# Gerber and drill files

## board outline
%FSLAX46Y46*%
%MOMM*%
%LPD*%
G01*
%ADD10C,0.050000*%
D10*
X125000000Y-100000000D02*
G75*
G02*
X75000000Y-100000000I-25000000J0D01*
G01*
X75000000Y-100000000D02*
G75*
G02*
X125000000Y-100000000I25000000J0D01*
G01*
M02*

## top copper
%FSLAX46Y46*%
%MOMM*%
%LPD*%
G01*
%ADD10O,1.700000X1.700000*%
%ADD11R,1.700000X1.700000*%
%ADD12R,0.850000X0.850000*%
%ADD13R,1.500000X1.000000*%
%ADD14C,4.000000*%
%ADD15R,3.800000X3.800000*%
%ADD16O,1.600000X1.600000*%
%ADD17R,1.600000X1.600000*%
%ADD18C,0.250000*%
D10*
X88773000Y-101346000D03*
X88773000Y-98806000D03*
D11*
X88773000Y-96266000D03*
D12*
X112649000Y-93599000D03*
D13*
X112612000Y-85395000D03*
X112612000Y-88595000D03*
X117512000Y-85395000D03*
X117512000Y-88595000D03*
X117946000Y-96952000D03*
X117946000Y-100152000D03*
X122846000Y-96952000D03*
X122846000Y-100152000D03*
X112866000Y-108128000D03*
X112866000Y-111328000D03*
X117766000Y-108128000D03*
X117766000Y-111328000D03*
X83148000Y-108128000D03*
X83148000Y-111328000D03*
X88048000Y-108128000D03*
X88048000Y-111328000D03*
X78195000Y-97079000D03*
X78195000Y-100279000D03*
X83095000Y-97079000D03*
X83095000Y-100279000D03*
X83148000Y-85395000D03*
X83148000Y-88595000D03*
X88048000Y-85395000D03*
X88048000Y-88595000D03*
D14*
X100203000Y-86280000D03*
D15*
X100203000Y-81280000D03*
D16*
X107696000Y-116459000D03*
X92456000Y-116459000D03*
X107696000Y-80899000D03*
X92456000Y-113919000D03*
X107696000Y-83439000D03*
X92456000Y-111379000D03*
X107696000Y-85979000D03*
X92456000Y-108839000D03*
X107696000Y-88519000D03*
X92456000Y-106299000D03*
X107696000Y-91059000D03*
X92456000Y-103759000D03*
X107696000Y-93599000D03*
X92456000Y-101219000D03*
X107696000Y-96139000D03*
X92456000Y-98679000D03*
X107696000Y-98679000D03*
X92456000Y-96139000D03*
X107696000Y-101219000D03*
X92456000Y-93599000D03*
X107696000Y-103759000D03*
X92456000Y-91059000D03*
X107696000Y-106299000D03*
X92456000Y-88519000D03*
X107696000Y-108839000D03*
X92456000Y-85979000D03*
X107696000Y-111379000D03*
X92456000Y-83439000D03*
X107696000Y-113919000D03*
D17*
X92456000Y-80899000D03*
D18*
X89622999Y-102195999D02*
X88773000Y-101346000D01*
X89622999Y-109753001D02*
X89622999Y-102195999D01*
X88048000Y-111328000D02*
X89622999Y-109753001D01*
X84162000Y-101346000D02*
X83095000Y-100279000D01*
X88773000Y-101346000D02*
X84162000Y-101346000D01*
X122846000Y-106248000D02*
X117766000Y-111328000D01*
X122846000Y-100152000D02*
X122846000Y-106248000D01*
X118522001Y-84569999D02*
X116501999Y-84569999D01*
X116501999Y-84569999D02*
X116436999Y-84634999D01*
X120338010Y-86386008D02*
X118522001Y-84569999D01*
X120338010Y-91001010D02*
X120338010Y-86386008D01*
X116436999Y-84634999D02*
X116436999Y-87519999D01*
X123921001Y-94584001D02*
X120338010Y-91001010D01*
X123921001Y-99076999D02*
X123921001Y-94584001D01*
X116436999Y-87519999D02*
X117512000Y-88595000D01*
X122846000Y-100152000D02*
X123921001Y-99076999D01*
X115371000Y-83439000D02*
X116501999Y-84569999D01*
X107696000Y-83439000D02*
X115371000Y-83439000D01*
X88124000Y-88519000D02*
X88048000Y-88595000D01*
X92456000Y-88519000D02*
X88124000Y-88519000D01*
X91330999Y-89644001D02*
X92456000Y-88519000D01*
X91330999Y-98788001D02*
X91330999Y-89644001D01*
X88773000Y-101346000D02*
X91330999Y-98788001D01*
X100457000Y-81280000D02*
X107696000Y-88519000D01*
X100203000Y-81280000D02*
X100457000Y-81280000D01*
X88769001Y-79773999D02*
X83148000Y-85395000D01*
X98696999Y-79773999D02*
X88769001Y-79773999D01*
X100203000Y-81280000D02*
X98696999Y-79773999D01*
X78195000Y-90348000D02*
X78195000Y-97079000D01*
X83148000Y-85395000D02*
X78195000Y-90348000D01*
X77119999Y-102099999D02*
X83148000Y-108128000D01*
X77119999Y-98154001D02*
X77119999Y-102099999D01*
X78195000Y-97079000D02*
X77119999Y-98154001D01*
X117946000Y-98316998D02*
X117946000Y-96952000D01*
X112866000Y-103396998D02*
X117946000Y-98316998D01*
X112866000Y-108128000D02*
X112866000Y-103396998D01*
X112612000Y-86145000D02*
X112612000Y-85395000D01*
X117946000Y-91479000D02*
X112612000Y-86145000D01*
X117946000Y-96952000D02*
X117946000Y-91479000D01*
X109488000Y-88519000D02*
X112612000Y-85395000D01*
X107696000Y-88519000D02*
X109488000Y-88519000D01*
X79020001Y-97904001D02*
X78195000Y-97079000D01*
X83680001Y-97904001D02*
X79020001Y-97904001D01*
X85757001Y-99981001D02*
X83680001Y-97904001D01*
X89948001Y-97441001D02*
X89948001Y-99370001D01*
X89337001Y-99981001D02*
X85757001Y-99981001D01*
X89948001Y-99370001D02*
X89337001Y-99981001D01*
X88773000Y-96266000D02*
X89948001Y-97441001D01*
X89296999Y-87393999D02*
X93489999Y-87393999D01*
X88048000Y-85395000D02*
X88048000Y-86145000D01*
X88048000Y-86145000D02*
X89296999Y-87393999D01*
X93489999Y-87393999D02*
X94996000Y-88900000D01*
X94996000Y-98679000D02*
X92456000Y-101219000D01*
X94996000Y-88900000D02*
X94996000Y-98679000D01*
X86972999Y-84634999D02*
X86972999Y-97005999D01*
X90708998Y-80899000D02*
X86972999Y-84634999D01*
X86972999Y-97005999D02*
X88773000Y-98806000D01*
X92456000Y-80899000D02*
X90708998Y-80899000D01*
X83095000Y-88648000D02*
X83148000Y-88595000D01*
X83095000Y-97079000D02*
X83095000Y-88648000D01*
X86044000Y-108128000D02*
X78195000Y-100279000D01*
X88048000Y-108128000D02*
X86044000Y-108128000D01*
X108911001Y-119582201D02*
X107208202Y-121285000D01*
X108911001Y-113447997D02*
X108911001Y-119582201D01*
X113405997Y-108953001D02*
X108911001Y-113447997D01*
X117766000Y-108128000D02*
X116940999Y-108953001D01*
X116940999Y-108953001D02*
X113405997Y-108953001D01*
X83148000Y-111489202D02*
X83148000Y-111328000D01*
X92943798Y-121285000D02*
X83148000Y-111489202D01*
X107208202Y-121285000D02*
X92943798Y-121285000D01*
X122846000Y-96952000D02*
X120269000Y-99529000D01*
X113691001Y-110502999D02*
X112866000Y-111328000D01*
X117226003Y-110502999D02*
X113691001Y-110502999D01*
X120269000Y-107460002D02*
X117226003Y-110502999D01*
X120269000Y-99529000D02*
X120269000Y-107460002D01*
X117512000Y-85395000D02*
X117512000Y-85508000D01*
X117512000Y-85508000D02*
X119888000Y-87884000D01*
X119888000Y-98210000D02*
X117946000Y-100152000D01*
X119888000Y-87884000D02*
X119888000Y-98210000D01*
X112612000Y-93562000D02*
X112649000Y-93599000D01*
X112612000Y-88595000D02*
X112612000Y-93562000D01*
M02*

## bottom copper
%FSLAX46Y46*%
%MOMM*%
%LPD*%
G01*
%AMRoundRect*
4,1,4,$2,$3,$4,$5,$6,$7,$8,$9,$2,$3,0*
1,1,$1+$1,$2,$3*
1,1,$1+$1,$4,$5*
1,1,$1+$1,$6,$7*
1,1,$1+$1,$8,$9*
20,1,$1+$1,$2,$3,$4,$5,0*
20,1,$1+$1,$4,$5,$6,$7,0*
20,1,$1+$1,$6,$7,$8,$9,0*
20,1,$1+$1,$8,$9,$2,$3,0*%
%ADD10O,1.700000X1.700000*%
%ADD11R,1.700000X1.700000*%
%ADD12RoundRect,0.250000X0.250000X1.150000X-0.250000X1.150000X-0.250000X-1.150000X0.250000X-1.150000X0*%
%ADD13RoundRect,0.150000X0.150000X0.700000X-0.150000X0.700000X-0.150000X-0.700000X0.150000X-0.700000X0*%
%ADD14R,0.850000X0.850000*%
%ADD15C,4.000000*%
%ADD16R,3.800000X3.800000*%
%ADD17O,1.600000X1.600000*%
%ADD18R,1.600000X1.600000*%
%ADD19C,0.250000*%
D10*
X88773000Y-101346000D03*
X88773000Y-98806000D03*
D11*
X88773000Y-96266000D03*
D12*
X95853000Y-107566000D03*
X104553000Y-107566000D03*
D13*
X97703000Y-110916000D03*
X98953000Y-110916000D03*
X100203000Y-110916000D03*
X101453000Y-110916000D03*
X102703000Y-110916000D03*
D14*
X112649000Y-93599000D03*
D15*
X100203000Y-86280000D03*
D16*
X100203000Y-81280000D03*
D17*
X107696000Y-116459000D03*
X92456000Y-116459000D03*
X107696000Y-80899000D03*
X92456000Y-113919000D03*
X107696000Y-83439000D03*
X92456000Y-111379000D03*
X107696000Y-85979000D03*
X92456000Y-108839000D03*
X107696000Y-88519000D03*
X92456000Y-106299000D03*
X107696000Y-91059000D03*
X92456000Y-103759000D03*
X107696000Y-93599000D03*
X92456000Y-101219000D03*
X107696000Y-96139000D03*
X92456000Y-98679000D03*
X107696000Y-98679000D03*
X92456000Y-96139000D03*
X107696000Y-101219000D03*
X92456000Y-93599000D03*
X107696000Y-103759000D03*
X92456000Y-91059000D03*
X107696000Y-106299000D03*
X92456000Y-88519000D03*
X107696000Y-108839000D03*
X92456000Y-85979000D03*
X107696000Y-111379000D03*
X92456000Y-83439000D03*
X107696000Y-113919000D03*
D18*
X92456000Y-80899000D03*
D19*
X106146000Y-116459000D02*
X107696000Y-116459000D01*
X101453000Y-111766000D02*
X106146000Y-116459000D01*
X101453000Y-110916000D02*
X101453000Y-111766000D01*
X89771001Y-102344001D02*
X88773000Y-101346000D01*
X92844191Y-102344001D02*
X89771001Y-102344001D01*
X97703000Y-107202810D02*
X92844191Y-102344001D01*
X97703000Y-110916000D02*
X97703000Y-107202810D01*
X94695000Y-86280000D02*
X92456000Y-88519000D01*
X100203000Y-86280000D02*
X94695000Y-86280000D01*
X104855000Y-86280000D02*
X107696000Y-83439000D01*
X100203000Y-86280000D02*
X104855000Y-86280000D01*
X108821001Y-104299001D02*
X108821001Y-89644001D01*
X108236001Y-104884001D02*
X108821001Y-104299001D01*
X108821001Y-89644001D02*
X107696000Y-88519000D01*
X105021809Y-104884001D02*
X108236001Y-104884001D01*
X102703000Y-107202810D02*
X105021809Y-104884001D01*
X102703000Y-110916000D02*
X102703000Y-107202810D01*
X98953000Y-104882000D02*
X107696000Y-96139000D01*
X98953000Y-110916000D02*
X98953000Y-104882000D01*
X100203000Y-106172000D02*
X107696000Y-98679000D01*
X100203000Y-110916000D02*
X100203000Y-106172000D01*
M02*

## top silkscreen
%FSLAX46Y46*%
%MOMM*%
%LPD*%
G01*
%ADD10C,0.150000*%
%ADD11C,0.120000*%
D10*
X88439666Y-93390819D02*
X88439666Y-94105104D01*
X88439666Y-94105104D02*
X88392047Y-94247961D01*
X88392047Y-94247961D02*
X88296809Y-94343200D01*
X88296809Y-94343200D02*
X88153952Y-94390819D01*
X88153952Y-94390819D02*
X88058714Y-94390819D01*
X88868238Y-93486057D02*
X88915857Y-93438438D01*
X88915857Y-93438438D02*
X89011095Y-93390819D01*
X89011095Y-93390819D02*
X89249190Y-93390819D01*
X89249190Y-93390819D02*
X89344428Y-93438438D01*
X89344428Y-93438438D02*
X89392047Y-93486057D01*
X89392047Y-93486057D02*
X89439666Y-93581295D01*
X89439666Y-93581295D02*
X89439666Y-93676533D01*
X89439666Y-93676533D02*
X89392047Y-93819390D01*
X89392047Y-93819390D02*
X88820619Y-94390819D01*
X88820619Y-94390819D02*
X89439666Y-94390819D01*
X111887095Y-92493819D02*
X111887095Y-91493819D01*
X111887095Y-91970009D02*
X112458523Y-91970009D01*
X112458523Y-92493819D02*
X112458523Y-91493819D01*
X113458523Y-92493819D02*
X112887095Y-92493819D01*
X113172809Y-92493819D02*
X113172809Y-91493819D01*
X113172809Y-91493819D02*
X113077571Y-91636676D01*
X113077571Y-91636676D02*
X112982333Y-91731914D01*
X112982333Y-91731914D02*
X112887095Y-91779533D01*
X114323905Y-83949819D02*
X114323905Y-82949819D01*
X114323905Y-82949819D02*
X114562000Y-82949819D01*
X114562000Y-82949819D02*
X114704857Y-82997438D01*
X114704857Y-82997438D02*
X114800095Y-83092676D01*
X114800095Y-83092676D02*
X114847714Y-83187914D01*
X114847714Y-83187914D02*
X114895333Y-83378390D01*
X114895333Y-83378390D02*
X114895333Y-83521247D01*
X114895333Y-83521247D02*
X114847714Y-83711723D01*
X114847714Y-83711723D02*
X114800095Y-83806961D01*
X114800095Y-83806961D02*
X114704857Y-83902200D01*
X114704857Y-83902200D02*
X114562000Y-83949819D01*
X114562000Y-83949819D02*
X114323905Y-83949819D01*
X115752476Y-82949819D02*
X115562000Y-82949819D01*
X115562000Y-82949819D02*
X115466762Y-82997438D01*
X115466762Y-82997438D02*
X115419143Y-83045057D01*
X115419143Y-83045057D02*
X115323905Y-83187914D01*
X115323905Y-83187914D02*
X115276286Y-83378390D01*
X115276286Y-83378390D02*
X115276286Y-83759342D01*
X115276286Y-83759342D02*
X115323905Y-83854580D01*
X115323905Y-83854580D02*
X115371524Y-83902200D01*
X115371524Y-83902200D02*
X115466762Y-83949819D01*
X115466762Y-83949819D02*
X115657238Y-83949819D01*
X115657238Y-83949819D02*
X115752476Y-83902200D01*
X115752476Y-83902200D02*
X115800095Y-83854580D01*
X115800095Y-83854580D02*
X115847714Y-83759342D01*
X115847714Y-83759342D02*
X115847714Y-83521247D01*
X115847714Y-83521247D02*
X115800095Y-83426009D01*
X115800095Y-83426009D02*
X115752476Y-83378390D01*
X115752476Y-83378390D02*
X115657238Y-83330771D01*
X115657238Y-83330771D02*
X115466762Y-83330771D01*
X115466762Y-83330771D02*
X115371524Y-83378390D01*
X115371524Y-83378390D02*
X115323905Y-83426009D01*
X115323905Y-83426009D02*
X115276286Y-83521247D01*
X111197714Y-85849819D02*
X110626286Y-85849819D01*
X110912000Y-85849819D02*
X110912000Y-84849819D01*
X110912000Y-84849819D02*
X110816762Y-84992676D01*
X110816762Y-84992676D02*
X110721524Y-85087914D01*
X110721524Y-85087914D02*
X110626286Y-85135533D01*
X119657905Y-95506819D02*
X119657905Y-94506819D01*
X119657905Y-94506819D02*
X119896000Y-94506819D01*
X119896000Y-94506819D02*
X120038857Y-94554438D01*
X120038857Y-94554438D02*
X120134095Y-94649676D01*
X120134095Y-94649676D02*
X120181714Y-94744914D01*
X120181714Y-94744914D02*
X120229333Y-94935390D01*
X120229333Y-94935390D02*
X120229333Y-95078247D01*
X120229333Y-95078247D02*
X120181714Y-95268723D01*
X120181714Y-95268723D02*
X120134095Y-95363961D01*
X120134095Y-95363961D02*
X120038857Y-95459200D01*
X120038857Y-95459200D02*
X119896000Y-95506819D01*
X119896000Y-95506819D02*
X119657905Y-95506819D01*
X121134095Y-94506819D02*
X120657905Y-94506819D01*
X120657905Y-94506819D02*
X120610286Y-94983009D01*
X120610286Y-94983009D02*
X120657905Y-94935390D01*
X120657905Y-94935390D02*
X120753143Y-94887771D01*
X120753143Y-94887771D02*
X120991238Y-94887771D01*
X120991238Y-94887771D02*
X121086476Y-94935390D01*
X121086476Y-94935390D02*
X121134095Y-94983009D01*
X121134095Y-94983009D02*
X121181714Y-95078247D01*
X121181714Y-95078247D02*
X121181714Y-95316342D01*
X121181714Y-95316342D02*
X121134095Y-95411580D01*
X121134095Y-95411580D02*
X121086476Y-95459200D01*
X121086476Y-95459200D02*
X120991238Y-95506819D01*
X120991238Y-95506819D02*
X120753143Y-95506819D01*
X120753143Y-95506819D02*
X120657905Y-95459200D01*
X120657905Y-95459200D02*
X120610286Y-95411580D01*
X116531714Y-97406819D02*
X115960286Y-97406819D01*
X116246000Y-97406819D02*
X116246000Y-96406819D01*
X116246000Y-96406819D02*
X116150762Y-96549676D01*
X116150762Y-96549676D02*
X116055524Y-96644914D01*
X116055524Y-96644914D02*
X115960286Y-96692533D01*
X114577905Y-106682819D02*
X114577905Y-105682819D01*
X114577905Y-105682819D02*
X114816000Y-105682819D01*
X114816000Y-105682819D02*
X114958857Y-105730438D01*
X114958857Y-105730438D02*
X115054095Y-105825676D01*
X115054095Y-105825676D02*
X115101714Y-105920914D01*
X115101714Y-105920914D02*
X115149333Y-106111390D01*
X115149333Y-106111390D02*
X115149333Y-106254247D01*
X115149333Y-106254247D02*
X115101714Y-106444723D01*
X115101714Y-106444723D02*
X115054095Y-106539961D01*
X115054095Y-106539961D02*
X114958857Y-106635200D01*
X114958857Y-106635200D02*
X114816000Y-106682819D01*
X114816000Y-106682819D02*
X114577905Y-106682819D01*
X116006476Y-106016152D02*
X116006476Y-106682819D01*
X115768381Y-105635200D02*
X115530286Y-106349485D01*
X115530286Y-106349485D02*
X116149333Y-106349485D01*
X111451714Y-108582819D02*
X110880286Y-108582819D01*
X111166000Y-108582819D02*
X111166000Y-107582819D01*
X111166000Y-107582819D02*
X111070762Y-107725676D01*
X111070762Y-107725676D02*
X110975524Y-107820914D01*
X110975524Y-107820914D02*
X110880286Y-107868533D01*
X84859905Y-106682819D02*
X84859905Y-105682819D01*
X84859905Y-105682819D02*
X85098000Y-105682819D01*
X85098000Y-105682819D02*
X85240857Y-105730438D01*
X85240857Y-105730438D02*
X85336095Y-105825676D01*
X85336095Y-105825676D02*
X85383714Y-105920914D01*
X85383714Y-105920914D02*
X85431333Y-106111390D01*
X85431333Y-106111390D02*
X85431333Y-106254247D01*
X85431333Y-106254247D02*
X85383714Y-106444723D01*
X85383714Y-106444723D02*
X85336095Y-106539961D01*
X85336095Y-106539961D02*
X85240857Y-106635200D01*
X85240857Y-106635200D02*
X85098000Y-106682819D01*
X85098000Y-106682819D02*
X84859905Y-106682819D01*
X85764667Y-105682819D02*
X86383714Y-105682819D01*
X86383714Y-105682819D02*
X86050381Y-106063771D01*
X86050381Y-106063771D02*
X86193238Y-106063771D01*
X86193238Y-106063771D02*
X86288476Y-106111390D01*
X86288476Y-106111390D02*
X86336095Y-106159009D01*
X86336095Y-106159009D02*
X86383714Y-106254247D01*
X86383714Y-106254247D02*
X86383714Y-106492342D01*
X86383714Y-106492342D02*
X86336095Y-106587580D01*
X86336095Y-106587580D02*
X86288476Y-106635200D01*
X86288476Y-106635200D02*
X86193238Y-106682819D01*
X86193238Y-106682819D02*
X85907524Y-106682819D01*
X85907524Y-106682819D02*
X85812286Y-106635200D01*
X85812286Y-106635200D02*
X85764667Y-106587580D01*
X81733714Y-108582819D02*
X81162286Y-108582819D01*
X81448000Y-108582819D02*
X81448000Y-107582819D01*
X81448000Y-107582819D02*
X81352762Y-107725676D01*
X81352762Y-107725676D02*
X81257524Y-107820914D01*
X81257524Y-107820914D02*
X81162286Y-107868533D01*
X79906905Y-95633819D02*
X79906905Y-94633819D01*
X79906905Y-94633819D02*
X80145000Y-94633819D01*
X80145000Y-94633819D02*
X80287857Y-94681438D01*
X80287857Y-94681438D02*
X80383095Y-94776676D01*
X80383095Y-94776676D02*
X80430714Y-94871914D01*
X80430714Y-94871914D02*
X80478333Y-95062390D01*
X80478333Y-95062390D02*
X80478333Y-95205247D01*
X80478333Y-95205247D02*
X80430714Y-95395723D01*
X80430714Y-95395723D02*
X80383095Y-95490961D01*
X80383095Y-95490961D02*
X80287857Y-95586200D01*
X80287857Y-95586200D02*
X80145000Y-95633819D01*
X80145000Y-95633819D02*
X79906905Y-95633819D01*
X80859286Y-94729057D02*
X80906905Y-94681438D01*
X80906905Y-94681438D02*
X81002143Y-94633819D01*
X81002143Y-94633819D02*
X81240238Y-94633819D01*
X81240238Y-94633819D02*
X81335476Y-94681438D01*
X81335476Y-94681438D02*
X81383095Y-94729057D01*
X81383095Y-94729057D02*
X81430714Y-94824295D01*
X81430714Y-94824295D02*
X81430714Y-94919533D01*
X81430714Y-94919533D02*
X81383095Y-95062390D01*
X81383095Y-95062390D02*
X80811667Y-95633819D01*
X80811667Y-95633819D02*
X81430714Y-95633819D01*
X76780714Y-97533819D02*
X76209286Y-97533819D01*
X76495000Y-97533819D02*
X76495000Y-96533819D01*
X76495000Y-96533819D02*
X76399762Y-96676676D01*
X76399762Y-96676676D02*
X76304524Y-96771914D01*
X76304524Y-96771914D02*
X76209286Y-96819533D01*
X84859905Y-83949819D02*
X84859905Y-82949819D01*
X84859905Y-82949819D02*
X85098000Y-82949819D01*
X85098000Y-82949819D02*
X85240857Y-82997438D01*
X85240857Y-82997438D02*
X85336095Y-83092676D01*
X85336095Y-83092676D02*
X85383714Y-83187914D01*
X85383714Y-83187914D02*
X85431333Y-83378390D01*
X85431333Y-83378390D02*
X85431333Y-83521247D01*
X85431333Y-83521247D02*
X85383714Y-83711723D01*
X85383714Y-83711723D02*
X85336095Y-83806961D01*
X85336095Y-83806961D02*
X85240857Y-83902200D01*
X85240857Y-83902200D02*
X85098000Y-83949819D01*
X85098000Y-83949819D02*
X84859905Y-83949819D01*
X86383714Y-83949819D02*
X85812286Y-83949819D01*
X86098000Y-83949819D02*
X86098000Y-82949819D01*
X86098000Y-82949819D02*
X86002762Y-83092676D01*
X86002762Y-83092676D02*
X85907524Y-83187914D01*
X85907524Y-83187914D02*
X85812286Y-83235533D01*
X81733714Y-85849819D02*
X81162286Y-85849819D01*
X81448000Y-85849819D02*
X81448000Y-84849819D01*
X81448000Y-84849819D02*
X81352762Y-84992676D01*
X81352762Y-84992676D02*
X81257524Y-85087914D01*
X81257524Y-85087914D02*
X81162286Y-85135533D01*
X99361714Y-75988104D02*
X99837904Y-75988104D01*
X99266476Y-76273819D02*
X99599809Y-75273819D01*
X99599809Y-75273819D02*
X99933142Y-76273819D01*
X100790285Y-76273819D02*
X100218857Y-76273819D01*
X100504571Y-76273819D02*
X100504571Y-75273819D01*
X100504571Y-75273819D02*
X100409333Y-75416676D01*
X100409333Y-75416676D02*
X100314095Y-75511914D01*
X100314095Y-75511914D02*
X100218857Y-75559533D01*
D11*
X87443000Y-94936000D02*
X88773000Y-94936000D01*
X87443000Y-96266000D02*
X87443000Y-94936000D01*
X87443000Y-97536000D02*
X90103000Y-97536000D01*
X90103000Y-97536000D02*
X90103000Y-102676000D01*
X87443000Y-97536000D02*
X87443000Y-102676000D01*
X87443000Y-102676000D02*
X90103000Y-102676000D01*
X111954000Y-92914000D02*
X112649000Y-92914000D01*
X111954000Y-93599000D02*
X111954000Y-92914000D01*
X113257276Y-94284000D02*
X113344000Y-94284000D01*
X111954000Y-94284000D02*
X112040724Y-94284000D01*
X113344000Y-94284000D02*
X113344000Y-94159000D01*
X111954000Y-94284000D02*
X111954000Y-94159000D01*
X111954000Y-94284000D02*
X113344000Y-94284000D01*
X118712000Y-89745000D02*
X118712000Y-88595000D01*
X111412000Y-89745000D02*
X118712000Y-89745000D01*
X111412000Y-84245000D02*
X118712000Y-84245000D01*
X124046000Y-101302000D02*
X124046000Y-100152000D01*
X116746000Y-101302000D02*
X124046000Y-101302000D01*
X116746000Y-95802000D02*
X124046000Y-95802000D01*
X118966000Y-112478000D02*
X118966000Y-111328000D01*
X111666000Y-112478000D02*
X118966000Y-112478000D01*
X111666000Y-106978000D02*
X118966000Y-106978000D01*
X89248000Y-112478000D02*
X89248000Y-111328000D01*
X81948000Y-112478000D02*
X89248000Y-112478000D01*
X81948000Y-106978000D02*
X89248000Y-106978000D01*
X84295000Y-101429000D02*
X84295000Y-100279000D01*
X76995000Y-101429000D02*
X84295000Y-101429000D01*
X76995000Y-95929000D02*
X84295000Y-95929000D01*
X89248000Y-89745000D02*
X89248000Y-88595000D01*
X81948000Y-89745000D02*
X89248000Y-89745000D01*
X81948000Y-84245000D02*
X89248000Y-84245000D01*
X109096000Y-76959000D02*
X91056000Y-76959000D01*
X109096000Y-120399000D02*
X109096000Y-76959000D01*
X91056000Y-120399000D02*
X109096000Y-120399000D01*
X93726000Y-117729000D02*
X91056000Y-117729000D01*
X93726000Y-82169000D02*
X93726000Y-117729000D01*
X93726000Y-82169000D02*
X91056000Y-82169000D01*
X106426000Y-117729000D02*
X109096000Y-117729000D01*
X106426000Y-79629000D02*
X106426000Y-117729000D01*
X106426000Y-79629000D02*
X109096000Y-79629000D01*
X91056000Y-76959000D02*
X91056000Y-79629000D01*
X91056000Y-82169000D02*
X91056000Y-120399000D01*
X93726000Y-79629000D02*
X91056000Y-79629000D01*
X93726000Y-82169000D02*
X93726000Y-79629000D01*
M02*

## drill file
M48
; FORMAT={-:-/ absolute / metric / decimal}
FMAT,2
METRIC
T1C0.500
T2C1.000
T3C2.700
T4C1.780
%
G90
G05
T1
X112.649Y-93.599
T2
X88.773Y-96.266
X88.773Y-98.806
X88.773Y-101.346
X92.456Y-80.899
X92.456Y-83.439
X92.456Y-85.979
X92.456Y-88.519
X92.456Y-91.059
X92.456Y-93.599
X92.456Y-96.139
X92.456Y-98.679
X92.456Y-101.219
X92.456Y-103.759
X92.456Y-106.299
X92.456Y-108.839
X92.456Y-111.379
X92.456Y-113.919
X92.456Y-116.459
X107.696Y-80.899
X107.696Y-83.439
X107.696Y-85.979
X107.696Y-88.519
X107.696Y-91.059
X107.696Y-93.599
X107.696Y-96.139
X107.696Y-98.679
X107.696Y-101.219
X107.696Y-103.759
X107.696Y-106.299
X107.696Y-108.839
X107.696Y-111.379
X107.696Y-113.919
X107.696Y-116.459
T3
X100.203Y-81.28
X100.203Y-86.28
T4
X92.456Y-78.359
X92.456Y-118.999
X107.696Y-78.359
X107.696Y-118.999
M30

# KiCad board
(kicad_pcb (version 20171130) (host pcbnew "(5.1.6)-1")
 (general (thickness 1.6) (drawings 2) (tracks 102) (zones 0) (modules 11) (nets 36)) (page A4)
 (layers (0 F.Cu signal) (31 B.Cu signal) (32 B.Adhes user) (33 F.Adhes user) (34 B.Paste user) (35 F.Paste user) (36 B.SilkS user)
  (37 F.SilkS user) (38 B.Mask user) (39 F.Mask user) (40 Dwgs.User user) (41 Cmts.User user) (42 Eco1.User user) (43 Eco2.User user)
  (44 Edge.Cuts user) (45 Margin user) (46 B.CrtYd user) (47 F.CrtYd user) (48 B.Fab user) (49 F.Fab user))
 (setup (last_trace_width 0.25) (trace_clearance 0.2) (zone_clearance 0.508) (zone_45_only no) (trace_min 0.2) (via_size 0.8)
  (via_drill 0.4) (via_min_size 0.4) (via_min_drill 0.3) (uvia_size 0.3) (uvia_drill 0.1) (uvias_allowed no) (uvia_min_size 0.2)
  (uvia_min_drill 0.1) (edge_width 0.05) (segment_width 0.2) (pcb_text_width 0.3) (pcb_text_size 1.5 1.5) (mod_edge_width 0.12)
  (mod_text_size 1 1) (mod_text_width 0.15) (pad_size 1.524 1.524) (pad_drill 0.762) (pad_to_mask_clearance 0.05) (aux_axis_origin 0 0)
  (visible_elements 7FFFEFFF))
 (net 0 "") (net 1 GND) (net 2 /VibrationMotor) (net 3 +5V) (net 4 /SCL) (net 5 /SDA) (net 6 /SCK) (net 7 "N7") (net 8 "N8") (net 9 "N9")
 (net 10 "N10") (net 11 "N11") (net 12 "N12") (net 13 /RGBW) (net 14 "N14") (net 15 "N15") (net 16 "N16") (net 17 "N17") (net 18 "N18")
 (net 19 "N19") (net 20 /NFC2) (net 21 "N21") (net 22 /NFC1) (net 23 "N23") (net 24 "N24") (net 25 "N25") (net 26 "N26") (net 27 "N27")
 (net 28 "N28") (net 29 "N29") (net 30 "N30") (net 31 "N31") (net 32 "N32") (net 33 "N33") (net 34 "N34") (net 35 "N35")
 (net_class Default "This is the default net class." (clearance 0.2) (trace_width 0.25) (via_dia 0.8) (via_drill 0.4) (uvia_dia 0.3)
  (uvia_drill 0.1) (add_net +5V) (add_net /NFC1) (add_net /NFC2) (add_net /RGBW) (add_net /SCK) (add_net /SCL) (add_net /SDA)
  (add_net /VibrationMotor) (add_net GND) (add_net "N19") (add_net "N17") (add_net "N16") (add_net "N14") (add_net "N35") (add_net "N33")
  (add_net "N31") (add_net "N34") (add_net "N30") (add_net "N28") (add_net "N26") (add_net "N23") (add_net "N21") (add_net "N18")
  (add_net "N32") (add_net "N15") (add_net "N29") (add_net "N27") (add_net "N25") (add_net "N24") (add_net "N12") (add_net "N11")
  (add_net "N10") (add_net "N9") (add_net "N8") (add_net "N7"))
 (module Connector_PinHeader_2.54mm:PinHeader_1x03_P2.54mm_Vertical (layer F.Cu) (at 88.773 96.266)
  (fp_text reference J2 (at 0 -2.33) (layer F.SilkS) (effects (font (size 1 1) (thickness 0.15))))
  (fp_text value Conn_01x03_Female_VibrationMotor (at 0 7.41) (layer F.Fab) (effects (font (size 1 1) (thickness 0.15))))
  (fp_line (start -1.33 -1.33) (end 0 -1.33) (layer F.SilkS) (width 0.12))
  (fp_line (start -1.33 0) (end -1.33 -1.33) (layer F.SilkS) (width 0.12))
  (fp_line (start -1.33 1.27) (end 1.33 1.27) (layer F.SilkS) (width 0.12))
  (fp_line (start 1.33 1.27) (end 1.33 6.41) (layer F.SilkS) (width 0.12))
  (fp_line (start -1.33 1.27) (end -1.33 6.41) (layer F.SilkS) (width 0.12))
  (fp_line (start -1.33 6.41) (end 1.33 6.41) (layer F.SilkS) (width 0.12))
  (pad 3 thru_hole oval (at 0 5.08) (size 1.7 1.7) (drill 1) (layers *.Cu *.Mask) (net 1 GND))
  (pad 2 thru_hole oval (at 0 2.54) (size 1.7 1.7) (drill 1) (layers *.Cu *.Mask) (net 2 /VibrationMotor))
  (pad 1 thru_hole rect (at 0 0) (size 1.7 1.7) (drill 1) (layers *.Cu *.Mask) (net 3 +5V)))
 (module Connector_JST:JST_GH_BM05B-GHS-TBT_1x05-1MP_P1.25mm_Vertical (layer B.Cu) (at 100.203 108.966 180)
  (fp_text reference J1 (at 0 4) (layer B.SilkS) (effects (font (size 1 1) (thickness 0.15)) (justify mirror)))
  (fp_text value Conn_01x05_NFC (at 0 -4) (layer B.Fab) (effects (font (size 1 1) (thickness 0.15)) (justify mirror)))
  (pad MP smd roundrect (at 4.35 1.4 180) (size 1 2.8) (layers B.Cu B.Paste B.Mask) (roundrect_rratio 0.25))
  (pad MP smd roundrect (at -4.35 1.4 180) (size 1 2.8) (layers B.Cu B.Paste B.Mask) (roundrect_rratio 0.25))
  (pad 5 smd roundrect (at 2.5 -1.95 180) (size 0.6 1.7) (layers B.Cu B.Paste B.Mask) (roundrect_rratio 0.25) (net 1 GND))
  (pad 4 smd roundrect (at 1.25 -1.95 180) (size 0.6 1.7) (layers B.Cu B.Paste B.Mask) (roundrect_rratio 0.25) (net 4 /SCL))
  (pad 3 smd roundrect (at 0 -1.95 180) (size 0.6 1.7) (layers B.Cu B.Paste B.Mask) (roundrect_rratio 0.25) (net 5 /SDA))
  (pad 2 smd roundrect (at -1.25 -1.95 180) (size 0.6 1.7) (layers B.Cu B.Paste B.Mask) (roundrect_rratio 0.25) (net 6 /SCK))
  (pad 1 smd roundrect (at -2.5 -1.95 180) (size 0.6 1.7) (layers B.Cu B.Paste B.Mask) (roundrect_rratio 0.25) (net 3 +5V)))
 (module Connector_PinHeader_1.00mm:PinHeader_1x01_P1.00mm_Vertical (layer F.Cu) (at 112.649 93.599)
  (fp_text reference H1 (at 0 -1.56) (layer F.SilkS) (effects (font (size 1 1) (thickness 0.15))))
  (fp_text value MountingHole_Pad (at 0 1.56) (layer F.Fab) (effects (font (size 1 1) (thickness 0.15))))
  (fp_line (start -0.695 -0.685) (end 0 -0.685) (layer F.SilkS) (width 0.12))
  (fp_line (start -0.695 0) (end -0.695 -0.685) (layer F.SilkS) (width 0.12))
  (fp_line (start 0.608276 0.685) (end 0.695 0.685) (layer F.SilkS) (width 0.12))
  (fp_line (start -0.695 0.685) (end -0.608276 0.685) (layer F.SilkS) (width 0.12))
  (fp_line (start 0.695 0.685) (end 0.695 0.56) (layer F.SilkS) (width 0.12))
  (fp_line (start -0.695 0.685) (end -0.695 0.56) (layer F.SilkS) (width 0.12))
  (fp_line (start -0.695 0.685) (end 0.695 0.685) (layer F.SilkS) (width 0.12))
  (pad 1 thru_hole rect (at 0 0) (size 0.85 0.85) (drill 0.5) (layers *.Cu *.Mask) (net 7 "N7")))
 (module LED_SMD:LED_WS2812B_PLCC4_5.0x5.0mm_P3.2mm (layer F.Cu) (at 115.062 86.995)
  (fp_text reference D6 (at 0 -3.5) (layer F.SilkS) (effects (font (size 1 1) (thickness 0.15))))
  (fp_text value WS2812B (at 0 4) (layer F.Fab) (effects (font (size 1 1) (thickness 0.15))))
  (fp_line (start 3.65 2.75) (end 3.65 1.6) (layer F.SilkS) (width 0.12))
  (fp_line (start -3.65 2.75) (end 3.65 2.75) (layer F.SilkS) (width 0.12))
  (fp_line (start -3.65 -2.75) (end 3.65 -2.75) (layer F.SilkS) (width 0.12))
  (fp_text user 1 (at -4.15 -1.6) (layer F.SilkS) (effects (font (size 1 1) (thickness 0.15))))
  (pad 1 smd rect (at -2.45 -1.6) (size 1.5 1) (layers F.Cu F.Paste F.Mask) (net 3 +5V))
  (pad 2 smd rect (at -2.45 1.6) (size 1.5 1) (layers F.Cu F.Paste F.Mask) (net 7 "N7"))
  (pad 4 smd rect (at 2.45 -1.6) (size 1.5 1) (layers F.Cu F.Paste F.Mask) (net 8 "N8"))
  (pad 3 smd rect (at 2.45 1.6) (size 1.5 1) (layers F.Cu F.Paste F.Mask) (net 1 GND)))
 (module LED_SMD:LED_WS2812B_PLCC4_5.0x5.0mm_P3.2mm (layer F.Cu) (at 120.396 98.552)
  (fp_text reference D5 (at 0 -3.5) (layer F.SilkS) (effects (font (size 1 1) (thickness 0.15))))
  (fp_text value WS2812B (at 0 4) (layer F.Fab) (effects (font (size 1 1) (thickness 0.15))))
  (fp_line (start 3.65 2.75) (end 3.65 1.6) (layer F.SilkS) (width 0.12))
  (fp_line (start -3.65 2.75) (end 3.65 2.75) (layer F.SilkS) (width 0.12))
  (fp_line (start -3.65 -2.75) (end 3.65 -2.75) (layer F.SilkS) (width 0.12))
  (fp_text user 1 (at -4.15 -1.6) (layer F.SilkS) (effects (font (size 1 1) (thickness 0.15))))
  (pad 1 smd rect (at -2.45 -1.6) (size 1.5 1) (layers F.Cu F.Paste F.Mask) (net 3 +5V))
  (pad 2 smd rect (at -2.45 1.6) (size 1.5 1) (layers F.Cu F.Paste F.Mask) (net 8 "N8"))
  (pad 4 smd rect (at 2.45 -1.6) (size 1.5 1) (layers F.Cu F.Paste F.Mask) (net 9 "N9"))
  (pad 3 smd rect (at 2.45 1.6) (size 1.5 1) (layers F.Cu F.Paste F.Mask) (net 1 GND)))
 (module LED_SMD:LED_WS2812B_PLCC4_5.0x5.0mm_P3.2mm (layer F.Cu) (at 115.316 109.728)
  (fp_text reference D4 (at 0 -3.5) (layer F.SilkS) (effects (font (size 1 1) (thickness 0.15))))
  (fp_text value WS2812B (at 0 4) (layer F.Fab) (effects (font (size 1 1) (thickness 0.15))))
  (fp_line (start 3.65 2.75) (end 3.65 1.6) (layer F.SilkS) (width 0.12))
  (fp_line (start -3.65 2.75) (end 3.65 2.75) (layer F.SilkS) (width 0.12))
  (fp_line (start -3.65 -2.75) (end 3.65 -2.75) (layer F.SilkS) (width 0.12))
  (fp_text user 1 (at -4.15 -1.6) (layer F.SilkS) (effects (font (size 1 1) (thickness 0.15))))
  (pad 1 smd rect (at -2.45 -1.6) (size 1.5 1) (layers F.Cu F.Paste F.Mask) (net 3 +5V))
  (pad 2 smd rect (at -2.45 1.6) (size 1.5 1) (layers F.Cu F.Paste F.Mask) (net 9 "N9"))
  (pad 4 smd rect (at 2.45 -1.6) (size 1.5 1) (layers F.Cu F.Paste F.Mask) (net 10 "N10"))
  (pad 3 smd rect (at 2.45 1.6) (size 1.5 1) (layers F.Cu F.Paste F.Mask) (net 1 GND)))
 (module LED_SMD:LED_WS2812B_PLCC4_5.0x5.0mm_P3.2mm (layer F.Cu) (at 85.598 109.728)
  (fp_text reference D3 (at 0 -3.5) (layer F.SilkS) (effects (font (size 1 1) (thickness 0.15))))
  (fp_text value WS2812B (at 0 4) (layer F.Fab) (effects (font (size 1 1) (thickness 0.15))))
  (fp_line (start 3.65 2.75) (end 3.65 1.6) (layer F.SilkS) (width 0.12))
  (fp_line (start -3.65 2.75) (end 3.65 2.75) (layer F.SilkS) (width 0.12))
  (fp_line (start -3.65 -2.75) (end 3.65 -2.75) (layer F.SilkS) (width 0.12))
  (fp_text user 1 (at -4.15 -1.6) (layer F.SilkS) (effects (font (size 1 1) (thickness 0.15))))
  (pad 1 smd rect (at -2.45 -1.6) (size 1.5 1) (layers F.Cu F.Paste F.Mask) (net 3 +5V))
  (pad 2 smd rect (at -2.45 1.6) (size 1.5 1) (layers F.Cu F.Paste F.Mask) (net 10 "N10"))
  (pad 4 smd rect (at 2.45 -1.6) (size 1.5 1) (layers F.Cu F.Paste F.Mask) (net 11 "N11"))
  (pad 3 smd rect (at 2.45 1.6) (size 1.5 1) (layers F.Cu F.Paste F.Mask) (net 1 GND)))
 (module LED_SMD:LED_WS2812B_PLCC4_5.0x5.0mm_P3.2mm (layer F.Cu) (at 80.645 98.679)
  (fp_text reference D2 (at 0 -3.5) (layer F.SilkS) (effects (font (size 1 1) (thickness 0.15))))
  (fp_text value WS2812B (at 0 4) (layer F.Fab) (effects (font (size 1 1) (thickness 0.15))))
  (fp_line (start 3.65 2.75) (end 3.65 1.6) (layer F.SilkS) (width 0.12))
  (fp_line (start -3.65 2.75) (end 3.65 2.75) (layer F.SilkS) (width 0.12))
  (fp_line (start -3.65 -2.75) (end 3.65 -2.75) (layer F.SilkS) (width 0.12))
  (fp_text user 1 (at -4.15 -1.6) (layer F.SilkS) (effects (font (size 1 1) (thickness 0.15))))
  (pad 1 smd rect (at -2.45 -1.6) (size 1.5 1) (layers F.Cu F.Paste F.Mask) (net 3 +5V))
  (pad 2 smd rect (at -2.45 1.6) (size 1.5 1) (layers F.Cu F.Paste F.Mask) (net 11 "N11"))
  (pad 4 smd rect (at 2.45 -1.6) (size 1.5 1) (layers F.Cu F.Paste F.Mask) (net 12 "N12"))
  (pad 3 smd rect (at 2.45 1.6) (size 1.5 1) (layers F.Cu F.Paste F.Mask) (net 1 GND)))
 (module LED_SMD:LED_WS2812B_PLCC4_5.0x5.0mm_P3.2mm (layer F.Cu) (at 85.598 86.995)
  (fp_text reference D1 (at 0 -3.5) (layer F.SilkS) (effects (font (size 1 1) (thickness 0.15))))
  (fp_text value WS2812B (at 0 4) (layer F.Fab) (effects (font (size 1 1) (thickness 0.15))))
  (fp_line (start 3.65 2.75) (end 3.65 1.6) (layer F.SilkS) (width 0.12))
  (fp_line (start -3.65 2.75) (end 3.65 2.75) (layer F.SilkS) (width 0.12))
  (fp_line (start -3.65 -2.75) (end 3.65 -2.75) (layer F.SilkS) (width 0.12))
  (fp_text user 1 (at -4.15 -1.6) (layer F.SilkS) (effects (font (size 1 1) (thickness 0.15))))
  (pad 1 smd rect (at -2.45 -1.6) (size 1.5 1) (layers F.Cu F.Paste F.Mask) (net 3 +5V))
  (pad 2 smd rect (at -2.45 1.6) (size 1.5 1) (layers F.Cu F.Paste F.Mask) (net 12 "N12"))
  (pad 4 smd rect (at 2.45 -1.6) (size 1.5 1) (layers F.Cu F.Paste F.Mask) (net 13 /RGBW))
  (pad 3 smd rect (at 2.45 1.6) (size 1.5 1) (layers F.Cu F.Paste F.Mask) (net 1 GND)))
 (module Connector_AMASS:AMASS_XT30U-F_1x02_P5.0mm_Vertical (layer B.Cu) (at 100.203 81.28 270)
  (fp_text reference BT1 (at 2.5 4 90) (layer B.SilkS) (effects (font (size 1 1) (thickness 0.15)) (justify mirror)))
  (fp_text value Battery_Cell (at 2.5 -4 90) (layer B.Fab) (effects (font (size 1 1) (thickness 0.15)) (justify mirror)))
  (pad 2 thru_hole circle (at 5 0 270) (size 4 4) (drill 2.7) (layers *.Cu *.Mask) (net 1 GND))
  (pad 1 thru_hole rect (at 0 0 270) (size 3.8 3.8) (drill 2.7) (layers *.Cu *.Mask) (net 3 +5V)))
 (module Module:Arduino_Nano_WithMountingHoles (layer F.Cu) (at 92.456 80.899)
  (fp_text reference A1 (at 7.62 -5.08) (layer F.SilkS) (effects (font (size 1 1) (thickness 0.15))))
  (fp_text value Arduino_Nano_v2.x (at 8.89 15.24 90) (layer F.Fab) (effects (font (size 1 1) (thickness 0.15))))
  (fp_line (start 16.64 -3.94) (end -1.4 -3.94) (layer F.SilkS) (width 0.12))
  (fp_line (start 16.64 39.5) (end 16.64 -3.94) (layer F.SilkS) (width 0.12))
  (fp_line (start -1.4 39.5) (end 16.64 39.5) (layer F.SilkS) (width 0.12))
  (fp_line (start 1.27 36.83) (end -1.4 36.83) (layer F.SilkS) (width 0.12))
  (fp_line (start 1.27 1.27) (end 1.27 36.83) (layer F.SilkS) (width 0.12))
  (fp_line (start 1.27 1.27) (end -1.4 1.27) (layer F.SilkS) (width 0.12))
  (fp_line (start 13.97 36.83) (end 16.64 36.83) (layer F.SilkS) (width 0.12))
  (fp_line (start 13.97 -1.27) (end 13.97 36.83) (layer F.SilkS) (width 0.12))
  (fp_line (start 13.97 -1.27) (end 16.64 -1.27) (layer F.SilkS) (width 0.12))
  (fp_line (start -1.4 -3.94) (end -1.4 -1.27) (layer F.SilkS) (width 0.12))
  (fp_line (start -1.4 1.27) (end -1.4 39.5) (layer F.SilkS) (width 0.12))
  (fp_line (start 1.27 -1.27) (end -1.4 -1.27) (layer F.SilkS) (width 0.12))
  (fp_line (start 1.27 1.27) (end 1.27 -1.27) (layer F.SilkS) (width 0.12))
  (pad "" np_thru_hole circle (at 0 38.1) (size 1.78 1.78) (drill 1.78) (layers *.Cu *.Mask))
  (pad "" np_thru_hole circle (at 15.24 38.1) (size 1.78 1.78) (drill 1.78) (layers *.Cu *.Mask))
  (pad "" np_thru_hole circle (at 15.24 -2.54) (size 1.78 1.78) (drill 1.78) (layers *.Cu *.Mask))
  (pad "" np_thru_hole circle (at 0 -2.54) (size 1.78 1.78) (drill 1.78) (layers *.Cu *.Mask))
  (pad 16 thru_hole oval (at 15.24 35.56) (size 1.6 1.6) (drill 1) (layers *.Cu *.Mask) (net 6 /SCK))
  (pad 15 thru_hole oval (at 0 35.56) (size 1.6 1.6) (drill 1) (layers *.Cu *.Mask) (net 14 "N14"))
  (pad 30 thru_hole oval (at 15.24 0) (size 1.6 1.6) (drill 1) (layers *.Cu *.Mask) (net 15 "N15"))
  (pad 14 thru_hole oval (at 0 33.02) (size 1.6 1.6) (drill 1) (layers *.Cu *.Mask) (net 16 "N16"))
  (pad 29 thru_hole oval (at 15.24 2.54) (size 1.6 1.6) (drill 1) (layers *.Cu *.Mask) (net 1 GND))
  (pad 13 thru_hole oval (at 0 30.48) (size 1.6 1.6) (drill 1) (layers *.Cu *.Mask) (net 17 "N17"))
  (pad 28 thru_hole oval (at 15.24 5.08) (size 1.6 1.6) (drill 1) (layers *.Cu *.Mask) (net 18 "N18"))
  (pad 12 thru_hole oval (at 0 27.94) (size 1.6 1.6) (drill 1) (layers *.Cu *.Mask) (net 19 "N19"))
  (pad 27 thru_hole oval (at 15.24 7.62) (size 1.6 1.6) (drill 1) (layers *.Cu *.Mask) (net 3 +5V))
  (pad 11 thru_hole oval (at 0 25.4) (size 1.6 1.6) (drill 1) (layers *.Cu *.Mask) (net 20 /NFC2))
  (pad 26 thru_hole oval (at 15.24 10.16) (size 1.6 1.6) (drill 1) (layers *.Cu *.Mask) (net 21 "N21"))
  (pad 10 thru_hole oval (at 0 22.86) (size 1.6 1.6) (drill 1) (layers *.Cu *.Mask) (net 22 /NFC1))
  (pad 25 thru_hole oval (at 15.24 12.7) (size 1.6 1.6) (drill 1) (layers *.Cu *.Mask) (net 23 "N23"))
  (pad 9 thru_hole oval (at 0 20.32) (size 1.6 1.6) (drill 1) (layers *.Cu *.Mask) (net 13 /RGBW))
  (pad 24 thru_hole oval (at 15.24 15.24) (size 1.6 1.6) (drill 1) (layers *.Cu *.Mask) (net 4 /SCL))
  (pad 8 thru_hole oval (at 0 17.78) (size 1.6 1.6) (drill 1) (layers *.Cu *.Mask) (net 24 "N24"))
  (pad 23 thru_hole oval (at 15.24 17.78) (size 1.6 1.6) (drill 1) (layers *.Cu *.Mask) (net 5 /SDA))
  (pad 7 thru_hole oval (at 0 15.24) (size 1.6 1.6) (drill 1) (layers *.Cu *.Mask) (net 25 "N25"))
  (pad 22 thru_hole oval (at 15.24 20.32) (size 1.6 1.6) (drill 1) (layers *.Cu *.Mask) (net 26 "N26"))
  (pad 6 thru_hole oval (at 0 12.7) (size 1.6 1.6) (drill 1) (layers *.Cu *.Mask) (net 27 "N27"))
  (pad 21 thru_hole oval (at 15.24 22.86) (size 1.6 1.6) (drill 1) (layers *.Cu *.Mask) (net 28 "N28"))
  (pad 5 thru_hole oval (at 0 10.16) (size 1.6 1.6) (drill 1) (layers *.Cu *.Mask) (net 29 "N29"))
  (pad 20 thru_hole oval (at 15.24 25.4) (size 1.6 1.6) (drill 1) (layers *.Cu *.Mask) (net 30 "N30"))
  (pad 4 thru_hole oval (at 0 7.62) (size 1.6 1.6) (drill 1) (layers *.Cu *.Mask) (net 1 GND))
  (pad 19 thru_hole oval (at 15.24 27.94) (size 1.6 1.6) (drill 1) (layers *.Cu *.Mask) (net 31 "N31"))
  (pad 3 thru_hole oval (at 0 5.08) (size 1.6 1.6) (drill 1) (layers *.Cu *.Mask) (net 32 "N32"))
  (pad 18 thru_hole oval (at 15.24 30.48) (size 1.6 1.6) (drill 1) (layers *.Cu *.Mask) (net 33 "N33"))
  (pad 2 thru_hole oval (at 0 2.54) (size 1.6 1.6) (drill 1) (layers *.Cu *.Mask) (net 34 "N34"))
  (pad 17 thru_hole oval (at 15.24 33.02) (size 1.6 1.6) (drill 1) (layers *.Cu *.Mask) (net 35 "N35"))
  (pad 1 thru_hole rect (at 0 0) (size 1.6 1.6) (drill 1) (layers *.Cu *.Mask) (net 2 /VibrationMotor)))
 (gr_circle (center 100 100) (end 125 100) (layer Edge.Cuts) (width 0.05))
 (segment (start 106.146 116.459) (end 107.696 116.459) (width 0.25) (layer B.Cu) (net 6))
 (segment (start 101.453 111.766) (end 106.146 116.459) (width 0.25) (layer B.Cu) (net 6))
 (segment (start 101.453 110.916) (end 101.453 111.766) (width 0.25) (layer B.Cu) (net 6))
 (segment (start 89.622999 102.195999) (end 88.773 101.346) (width 0.25) (layer F.Cu) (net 1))
 (segment (start 89.622999 109.753001) (end 89.622999 102.195999) (width 0.25) (layer F.Cu) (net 1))
 (segment (start 88.048 111.328) (end 89.622999 109.753001) (width 0.25) (layer F.Cu) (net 1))
 (segment (start 84.162 101.346) (end 83.095 100.279) (width 0.25) (layer F.Cu) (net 1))
 (segment (start 88.773 101.346) (end 84.162 101.346) (width 0.25) (layer F.Cu) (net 1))
 (segment (start 122.846 106.248) (end 117.766 111.328) (width 0.25) (layer F.Cu) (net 1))
 (segment (start 122.846 100.152) (end 122.846 106.248) (width 0.25) (layer F.Cu) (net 1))
 (segment (start 118.522001 84.569999) (end 116.501999 84.569999) (width 0.25) (layer F.Cu) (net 1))
 (segment (start 116.501999 84.569999) (end 116.436999 84.634999) (width 0.25) (layer F.Cu) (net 1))
 (segment (start 120.33801 86.386008) (end 118.522001 84.569999) (width 0.25) (layer F.Cu) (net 1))
 (segment (start 120.33801 91.00101) (end 120.33801 86.386008) (width 0.25) (layer F.Cu) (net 1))
 (segment (start 116.436999 84.634999) (end 116.436999 87.519999) (width 0.25) (layer F.Cu) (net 1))
 (segment (start 123.921001 94.584001) (end 120.33801 91.00101) (width 0.25) (layer F.Cu) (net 1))
 (segment (start 123.921001 99.076999) (end 123.921001 94.584001) (width 0.25) (layer F.Cu) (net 1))
 (segment (start 116.436999 87.519999) (end 117.512 88.595) (width 0.25) (layer F.Cu) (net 1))
 (segment (start 122.846 100.152) (end 123.921001 99.076999) (width 0.25) (layer F.Cu) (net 1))
 (segment (start 115.371 83.439) (end 116.501999 84.569999) (width 0.25) (layer F.Cu) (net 1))
 (segment (start 107.696 83.439) (end 115.371 83.439) (width 0.25) (layer F.Cu) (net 1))
 (segment (start 89.771001 102.344001) (end 88.773 101.346) (width 0.25) (layer B.Cu) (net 1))
 (segment (start 92.844191 102.344001) (end 89.771001 102.344001) (width 0.25) (layer B.Cu) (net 1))
 (segment (start 97.703 107.20281) (end 92.844191 102.344001) (width 0.25) (layer B.Cu) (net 1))
 (segment (start 97.703 110.916) (end 97.703 107.20281) (width 0.25) (layer B.Cu) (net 1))
 (segment (start 94.695 86.28) (end 92.456 88.519) (width 0.25) (layer B.Cu) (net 1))
 (segment (start 100.203 86.28) (end 94.695 86.28) (width 0.25) (layer B.Cu) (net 1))
 (segment (start 104.855 86.28) (end 107.696 83.439) (width 0.25) (layer B.Cu) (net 1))
 (segment (start 100.203 86.28) (end 104.855 86.28) (width 0.25) (layer B.Cu) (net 1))
 (segment (start 88.124 88.519) (end 88.048 88.595) (width 0.25) (layer F.Cu) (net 1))
 (segment (start 92.456 88.519) (end 88.124 88.519) (width 0.25) (layer F.Cu) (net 1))
 (segment (start 91.330999 89.644001) (end 92.456 88.519) (width 0.25) (layer F.Cu) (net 1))
 (segment (start 91.330999 98.788001) (end 91.330999 89.644001) (width 0.25) (layer F.Cu) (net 1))
 (segment (start 88.773 101.346) (end 91.330999 98.788001) (width 0.25) (layer F.Cu) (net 1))
 (segment (start 100.457 81.28) (end 107.696 88.519) (width 0.25) (layer F.Cu) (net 3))
 (segment (start 100.203 81.28) (end 100.457 81.28) (width 0.25) (layer F.Cu) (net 3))
 (segment (start 88.769001 79.773999) (end 83.148 85.395) (width 0.25) (layer F.Cu) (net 3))
 (segment (start 98.696999 79.773999) (end 88.769001 79.773999) (width 0.25) (layer F.Cu) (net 3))
 (segment (start 100.203 81.28) (end 98.696999 79.773999) (width 0.25) (layer F.Cu) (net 3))
 (segment (start 78.195 90.348) (end 78.195 97.079) (width 0.25) (layer F.Cu) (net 3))
 (segment (start 83.148 85.395) (end 78.195 90.348) (width 0.25) (layer F.Cu) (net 3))
 (segment (start 77.119999 102.099999) (end 83.148 108.128) (width 0.25) (layer F.Cu) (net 3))
 (segment (start 77.119999 98.154001) (end 77.119999 102.099999) (width 0.25) (layer F.Cu) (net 3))
 (segment (start 78.195 97.079) (end 77.119999 98.154001) (width 0.25) (layer F.Cu) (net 3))
 (segment (start 117.946 98.316998) (end 117.946 96.952) (width 0.25) (layer F.Cu) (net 3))
 (segment (start 112.866 103.396998) (end 117.946 98.316998) (width 0.25) (layer F.Cu) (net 3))
 (segment (start 112.866 108.128) (end 112.866 103.396998) (width 0.25) (layer F.Cu) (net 3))
 (segment (start 112.612 86.145) (end 112.612 85.395) (width 0.25) (layer F.Cu) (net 3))
 (segment (start 117.946 91.479) (end 112.612 86.145) (width 0.25) (layer F.Cu) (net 3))
 (segment (start 117.946 96.952) (end 117.946 91.479) (width 0.25) (layer F.Cu) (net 3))
 (segment (start 109.488 88.519) (end 112.612 85.395) (width 0.25) (layer F.Cu) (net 3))
 (segment (start 107.696 88.519) (end 109.488 88.519) (width 0.25) (layer F.Cu) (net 3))
 (segment (start 108.821001 104.299001) (end 108.821001 89.644001) (width 0.25) (layer B.Cu) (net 3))
 (segment (start 108.236001 104.884001) (end 108.821001 104.299001) (width 0.25) (layer B.Cu) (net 3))
 (segment (start 108.821001 89.644001) (end 107.696 88.519) (width 0.25) (layer B.Cu) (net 3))
 (segment (start 105.021809 104.884001) (end 108.236001 104.884001) (width 0.25) (layer B.Cu) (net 3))
 (segment (start 102.703 107.20281) (end 105.021809 104.884001) (width 0.25) (layer B.Cu) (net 3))
 (segment (start 102.703 110.916) (end 102.703 107.20281) (width 0.25) (layer B.Cu) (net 3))
 (segment (start 79.020001 97.904001) (end 78.195 97.079) (width 0.25) (layer F.Cu) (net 3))
 (segment (start 83.680001 97.904001) (end 79.020001 97.904001) (width 0.25) (layer F.Cu) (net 3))
 (segment (start 85.757001 99.981001) (end 83.680001 97.904001) (width 0.25) (layer F.Cu) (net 3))
 (segment (start 89.948001 97.441001) (end 89.948001 99.370001) (width 0.25) (layer F.Cu) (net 3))
 (segment (start 89.337001 99.981001) (end 85.757001 99.981001) (width 0.25) (layer F.Cu) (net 3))
 (segment (start 89.948001 99.370001) (end 89.337001 99.981001) (width 0.25) (layer F.Cu) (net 3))
 (segment (start 88.773 96.266) (end 89.948001 97.441001) (width 0.25) (layer F.Cu) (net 3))
 (segment (start 89.296999 87.393999) (end 93.489999 87.393999) (width 0.25) (layer F.Cu) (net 13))
 (segment (start 88.048 85.395) (end 88.048 86.145) (width 0.25) (layer F.Cu) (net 13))
 (segment (start 88.048 86.145) (end 89.296999 87.393999) (width 0.25) (layer F.Cu) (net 13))
 (segment (start 93.489999 87.393999) (end 94.996 88.9) (width 0.25) (layer F.Cu) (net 13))
 (segment (start 94.996 98.679) (end 92.456 101.219) (width 0.25) (layer F.Cu) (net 13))
 (segment (start 94.996 88.9) (end 94.996 98.679) (width 0.25) (layer F.Cu) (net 13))
 (segment (start 98.953 104.882) (end 107.696 96.139) (width 0.25) (layer B.Cu) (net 4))
 (segment (start 98.953 110.916) (end 98.953 104.882) (width 0.25) (layer B.Cu) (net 4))
 (segment (start 100.203 106.172) (end 107.696 98.679) (width 0.25) (layer B.Cu) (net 5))
 (segment (start 100.203 110.916) (end 100.203 106.172) (width 0.25) (layer B.Cu) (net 5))
 (segment (start 86.972999 84.634999) (end 86.972999 97.005999) (width 0.25) (layer F.Cu) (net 2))
 (segment (start 90.708998 80.899) (end 86.972999 84.634999) (width 0.25) (layer F.Cu) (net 2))
 (segment (start 86.972999 97.005999) (end 88.773 98.806) (width 0.25) (layer F.Cu) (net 2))
 (segment (start 92.456 80.899) (end 90.708998 80.899) (width 0.25) (layer F.Cu) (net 2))
 (segment (start 83.095 88.648) (end 83.148 88.595) (width 0.25) (layer F.Cu) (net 12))
 (segment (start 83.095 97.079) (end 83.095 88.648) (width 0.25) (layer F.Cu) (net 12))
 (segment (start 86.044 108.128) (end 78.195 100.279) (width 0.25) (layer F.Cu) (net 11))
 (segment (start 88.048 108.128) (end 86.044 108.128) (width 0.25) (layer F.Cu) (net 11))
 (segment (start 108.911001 119.582201) (end 107.208202 121.285) (width 0.25) (layer F.Cu) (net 10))
 (segment (start 108.911001 113.447997) (end 108.911001 119.582201) (width 0.25) (layer F.Cu) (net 10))
 (segment (start 113.405997 108.953001) (end 108.911001 113.447997) (width 0.25) (layer F.Cu) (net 10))
 (segment (start 117.766 108.128) (end 116.940999 108.953001) (width 0.25) (layer F.Cu) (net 10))
 (segment (start 116.940999 108.953001) (end 113.405997 108.953001) (width 0.25) (layer F.Cu) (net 10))
 (segment (start 83.148 111.489202) (end 83.148 111.328) (width 0.25) (layer F.Cu) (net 10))
 (segment (start 92.943798 121.285) (end 83.148 111.489202) (width 0.25) (layer F.Cu) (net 10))
 (segment (start 107.208202 121.285) (end 92.943798 121.285) (width 0.25) (layer F.Cu) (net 10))
 (segment (start 122.846 96.952) (end 120.269 99.529) (width 0.25) (layer F.Cu) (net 9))
 (segment (start 113.691001 110.502999) (end 112.866 111.328) (width 0.25) (layer F.Cu) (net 9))
 (segment (start 117.226003 110.502999) (end 113.691001 110.502999) (width 0.25) (layer F.Cu) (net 9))
 (segment (start 120.269 107.460002) (end 117.226003 110.502999) (width 0.25) (layer F.Cu) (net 9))
 (segment (start 120.269 99.529) (end 120.269 107.460002) (width 0.25) (layer F.Cu) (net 9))
 (segment (start 117.512 85.395) (end 117.512 85.508) (width 0.25) (layer F.Cu) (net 8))
 (segment (start 117.512 85.508) (end 119.888 87.884) (width 0.25) (layer F.Cu) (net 8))
 (segment (start 119.888 98.21) (end 117.946 100.152) (width 0.25) (layer F.Cu) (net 8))
 (segment (start 119.888 87.884) (end 119.888 98.21) (width 0.25) (layer F.Cu) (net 8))
 (segment (start 112.612 93.562) (end 112.649 93.599) (width 0.25) (layer F.Cu) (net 7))
 (segment (start 112.612 88.595) (end 112.612 93.562) (width 0.25) (layer F.Cu) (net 7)))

